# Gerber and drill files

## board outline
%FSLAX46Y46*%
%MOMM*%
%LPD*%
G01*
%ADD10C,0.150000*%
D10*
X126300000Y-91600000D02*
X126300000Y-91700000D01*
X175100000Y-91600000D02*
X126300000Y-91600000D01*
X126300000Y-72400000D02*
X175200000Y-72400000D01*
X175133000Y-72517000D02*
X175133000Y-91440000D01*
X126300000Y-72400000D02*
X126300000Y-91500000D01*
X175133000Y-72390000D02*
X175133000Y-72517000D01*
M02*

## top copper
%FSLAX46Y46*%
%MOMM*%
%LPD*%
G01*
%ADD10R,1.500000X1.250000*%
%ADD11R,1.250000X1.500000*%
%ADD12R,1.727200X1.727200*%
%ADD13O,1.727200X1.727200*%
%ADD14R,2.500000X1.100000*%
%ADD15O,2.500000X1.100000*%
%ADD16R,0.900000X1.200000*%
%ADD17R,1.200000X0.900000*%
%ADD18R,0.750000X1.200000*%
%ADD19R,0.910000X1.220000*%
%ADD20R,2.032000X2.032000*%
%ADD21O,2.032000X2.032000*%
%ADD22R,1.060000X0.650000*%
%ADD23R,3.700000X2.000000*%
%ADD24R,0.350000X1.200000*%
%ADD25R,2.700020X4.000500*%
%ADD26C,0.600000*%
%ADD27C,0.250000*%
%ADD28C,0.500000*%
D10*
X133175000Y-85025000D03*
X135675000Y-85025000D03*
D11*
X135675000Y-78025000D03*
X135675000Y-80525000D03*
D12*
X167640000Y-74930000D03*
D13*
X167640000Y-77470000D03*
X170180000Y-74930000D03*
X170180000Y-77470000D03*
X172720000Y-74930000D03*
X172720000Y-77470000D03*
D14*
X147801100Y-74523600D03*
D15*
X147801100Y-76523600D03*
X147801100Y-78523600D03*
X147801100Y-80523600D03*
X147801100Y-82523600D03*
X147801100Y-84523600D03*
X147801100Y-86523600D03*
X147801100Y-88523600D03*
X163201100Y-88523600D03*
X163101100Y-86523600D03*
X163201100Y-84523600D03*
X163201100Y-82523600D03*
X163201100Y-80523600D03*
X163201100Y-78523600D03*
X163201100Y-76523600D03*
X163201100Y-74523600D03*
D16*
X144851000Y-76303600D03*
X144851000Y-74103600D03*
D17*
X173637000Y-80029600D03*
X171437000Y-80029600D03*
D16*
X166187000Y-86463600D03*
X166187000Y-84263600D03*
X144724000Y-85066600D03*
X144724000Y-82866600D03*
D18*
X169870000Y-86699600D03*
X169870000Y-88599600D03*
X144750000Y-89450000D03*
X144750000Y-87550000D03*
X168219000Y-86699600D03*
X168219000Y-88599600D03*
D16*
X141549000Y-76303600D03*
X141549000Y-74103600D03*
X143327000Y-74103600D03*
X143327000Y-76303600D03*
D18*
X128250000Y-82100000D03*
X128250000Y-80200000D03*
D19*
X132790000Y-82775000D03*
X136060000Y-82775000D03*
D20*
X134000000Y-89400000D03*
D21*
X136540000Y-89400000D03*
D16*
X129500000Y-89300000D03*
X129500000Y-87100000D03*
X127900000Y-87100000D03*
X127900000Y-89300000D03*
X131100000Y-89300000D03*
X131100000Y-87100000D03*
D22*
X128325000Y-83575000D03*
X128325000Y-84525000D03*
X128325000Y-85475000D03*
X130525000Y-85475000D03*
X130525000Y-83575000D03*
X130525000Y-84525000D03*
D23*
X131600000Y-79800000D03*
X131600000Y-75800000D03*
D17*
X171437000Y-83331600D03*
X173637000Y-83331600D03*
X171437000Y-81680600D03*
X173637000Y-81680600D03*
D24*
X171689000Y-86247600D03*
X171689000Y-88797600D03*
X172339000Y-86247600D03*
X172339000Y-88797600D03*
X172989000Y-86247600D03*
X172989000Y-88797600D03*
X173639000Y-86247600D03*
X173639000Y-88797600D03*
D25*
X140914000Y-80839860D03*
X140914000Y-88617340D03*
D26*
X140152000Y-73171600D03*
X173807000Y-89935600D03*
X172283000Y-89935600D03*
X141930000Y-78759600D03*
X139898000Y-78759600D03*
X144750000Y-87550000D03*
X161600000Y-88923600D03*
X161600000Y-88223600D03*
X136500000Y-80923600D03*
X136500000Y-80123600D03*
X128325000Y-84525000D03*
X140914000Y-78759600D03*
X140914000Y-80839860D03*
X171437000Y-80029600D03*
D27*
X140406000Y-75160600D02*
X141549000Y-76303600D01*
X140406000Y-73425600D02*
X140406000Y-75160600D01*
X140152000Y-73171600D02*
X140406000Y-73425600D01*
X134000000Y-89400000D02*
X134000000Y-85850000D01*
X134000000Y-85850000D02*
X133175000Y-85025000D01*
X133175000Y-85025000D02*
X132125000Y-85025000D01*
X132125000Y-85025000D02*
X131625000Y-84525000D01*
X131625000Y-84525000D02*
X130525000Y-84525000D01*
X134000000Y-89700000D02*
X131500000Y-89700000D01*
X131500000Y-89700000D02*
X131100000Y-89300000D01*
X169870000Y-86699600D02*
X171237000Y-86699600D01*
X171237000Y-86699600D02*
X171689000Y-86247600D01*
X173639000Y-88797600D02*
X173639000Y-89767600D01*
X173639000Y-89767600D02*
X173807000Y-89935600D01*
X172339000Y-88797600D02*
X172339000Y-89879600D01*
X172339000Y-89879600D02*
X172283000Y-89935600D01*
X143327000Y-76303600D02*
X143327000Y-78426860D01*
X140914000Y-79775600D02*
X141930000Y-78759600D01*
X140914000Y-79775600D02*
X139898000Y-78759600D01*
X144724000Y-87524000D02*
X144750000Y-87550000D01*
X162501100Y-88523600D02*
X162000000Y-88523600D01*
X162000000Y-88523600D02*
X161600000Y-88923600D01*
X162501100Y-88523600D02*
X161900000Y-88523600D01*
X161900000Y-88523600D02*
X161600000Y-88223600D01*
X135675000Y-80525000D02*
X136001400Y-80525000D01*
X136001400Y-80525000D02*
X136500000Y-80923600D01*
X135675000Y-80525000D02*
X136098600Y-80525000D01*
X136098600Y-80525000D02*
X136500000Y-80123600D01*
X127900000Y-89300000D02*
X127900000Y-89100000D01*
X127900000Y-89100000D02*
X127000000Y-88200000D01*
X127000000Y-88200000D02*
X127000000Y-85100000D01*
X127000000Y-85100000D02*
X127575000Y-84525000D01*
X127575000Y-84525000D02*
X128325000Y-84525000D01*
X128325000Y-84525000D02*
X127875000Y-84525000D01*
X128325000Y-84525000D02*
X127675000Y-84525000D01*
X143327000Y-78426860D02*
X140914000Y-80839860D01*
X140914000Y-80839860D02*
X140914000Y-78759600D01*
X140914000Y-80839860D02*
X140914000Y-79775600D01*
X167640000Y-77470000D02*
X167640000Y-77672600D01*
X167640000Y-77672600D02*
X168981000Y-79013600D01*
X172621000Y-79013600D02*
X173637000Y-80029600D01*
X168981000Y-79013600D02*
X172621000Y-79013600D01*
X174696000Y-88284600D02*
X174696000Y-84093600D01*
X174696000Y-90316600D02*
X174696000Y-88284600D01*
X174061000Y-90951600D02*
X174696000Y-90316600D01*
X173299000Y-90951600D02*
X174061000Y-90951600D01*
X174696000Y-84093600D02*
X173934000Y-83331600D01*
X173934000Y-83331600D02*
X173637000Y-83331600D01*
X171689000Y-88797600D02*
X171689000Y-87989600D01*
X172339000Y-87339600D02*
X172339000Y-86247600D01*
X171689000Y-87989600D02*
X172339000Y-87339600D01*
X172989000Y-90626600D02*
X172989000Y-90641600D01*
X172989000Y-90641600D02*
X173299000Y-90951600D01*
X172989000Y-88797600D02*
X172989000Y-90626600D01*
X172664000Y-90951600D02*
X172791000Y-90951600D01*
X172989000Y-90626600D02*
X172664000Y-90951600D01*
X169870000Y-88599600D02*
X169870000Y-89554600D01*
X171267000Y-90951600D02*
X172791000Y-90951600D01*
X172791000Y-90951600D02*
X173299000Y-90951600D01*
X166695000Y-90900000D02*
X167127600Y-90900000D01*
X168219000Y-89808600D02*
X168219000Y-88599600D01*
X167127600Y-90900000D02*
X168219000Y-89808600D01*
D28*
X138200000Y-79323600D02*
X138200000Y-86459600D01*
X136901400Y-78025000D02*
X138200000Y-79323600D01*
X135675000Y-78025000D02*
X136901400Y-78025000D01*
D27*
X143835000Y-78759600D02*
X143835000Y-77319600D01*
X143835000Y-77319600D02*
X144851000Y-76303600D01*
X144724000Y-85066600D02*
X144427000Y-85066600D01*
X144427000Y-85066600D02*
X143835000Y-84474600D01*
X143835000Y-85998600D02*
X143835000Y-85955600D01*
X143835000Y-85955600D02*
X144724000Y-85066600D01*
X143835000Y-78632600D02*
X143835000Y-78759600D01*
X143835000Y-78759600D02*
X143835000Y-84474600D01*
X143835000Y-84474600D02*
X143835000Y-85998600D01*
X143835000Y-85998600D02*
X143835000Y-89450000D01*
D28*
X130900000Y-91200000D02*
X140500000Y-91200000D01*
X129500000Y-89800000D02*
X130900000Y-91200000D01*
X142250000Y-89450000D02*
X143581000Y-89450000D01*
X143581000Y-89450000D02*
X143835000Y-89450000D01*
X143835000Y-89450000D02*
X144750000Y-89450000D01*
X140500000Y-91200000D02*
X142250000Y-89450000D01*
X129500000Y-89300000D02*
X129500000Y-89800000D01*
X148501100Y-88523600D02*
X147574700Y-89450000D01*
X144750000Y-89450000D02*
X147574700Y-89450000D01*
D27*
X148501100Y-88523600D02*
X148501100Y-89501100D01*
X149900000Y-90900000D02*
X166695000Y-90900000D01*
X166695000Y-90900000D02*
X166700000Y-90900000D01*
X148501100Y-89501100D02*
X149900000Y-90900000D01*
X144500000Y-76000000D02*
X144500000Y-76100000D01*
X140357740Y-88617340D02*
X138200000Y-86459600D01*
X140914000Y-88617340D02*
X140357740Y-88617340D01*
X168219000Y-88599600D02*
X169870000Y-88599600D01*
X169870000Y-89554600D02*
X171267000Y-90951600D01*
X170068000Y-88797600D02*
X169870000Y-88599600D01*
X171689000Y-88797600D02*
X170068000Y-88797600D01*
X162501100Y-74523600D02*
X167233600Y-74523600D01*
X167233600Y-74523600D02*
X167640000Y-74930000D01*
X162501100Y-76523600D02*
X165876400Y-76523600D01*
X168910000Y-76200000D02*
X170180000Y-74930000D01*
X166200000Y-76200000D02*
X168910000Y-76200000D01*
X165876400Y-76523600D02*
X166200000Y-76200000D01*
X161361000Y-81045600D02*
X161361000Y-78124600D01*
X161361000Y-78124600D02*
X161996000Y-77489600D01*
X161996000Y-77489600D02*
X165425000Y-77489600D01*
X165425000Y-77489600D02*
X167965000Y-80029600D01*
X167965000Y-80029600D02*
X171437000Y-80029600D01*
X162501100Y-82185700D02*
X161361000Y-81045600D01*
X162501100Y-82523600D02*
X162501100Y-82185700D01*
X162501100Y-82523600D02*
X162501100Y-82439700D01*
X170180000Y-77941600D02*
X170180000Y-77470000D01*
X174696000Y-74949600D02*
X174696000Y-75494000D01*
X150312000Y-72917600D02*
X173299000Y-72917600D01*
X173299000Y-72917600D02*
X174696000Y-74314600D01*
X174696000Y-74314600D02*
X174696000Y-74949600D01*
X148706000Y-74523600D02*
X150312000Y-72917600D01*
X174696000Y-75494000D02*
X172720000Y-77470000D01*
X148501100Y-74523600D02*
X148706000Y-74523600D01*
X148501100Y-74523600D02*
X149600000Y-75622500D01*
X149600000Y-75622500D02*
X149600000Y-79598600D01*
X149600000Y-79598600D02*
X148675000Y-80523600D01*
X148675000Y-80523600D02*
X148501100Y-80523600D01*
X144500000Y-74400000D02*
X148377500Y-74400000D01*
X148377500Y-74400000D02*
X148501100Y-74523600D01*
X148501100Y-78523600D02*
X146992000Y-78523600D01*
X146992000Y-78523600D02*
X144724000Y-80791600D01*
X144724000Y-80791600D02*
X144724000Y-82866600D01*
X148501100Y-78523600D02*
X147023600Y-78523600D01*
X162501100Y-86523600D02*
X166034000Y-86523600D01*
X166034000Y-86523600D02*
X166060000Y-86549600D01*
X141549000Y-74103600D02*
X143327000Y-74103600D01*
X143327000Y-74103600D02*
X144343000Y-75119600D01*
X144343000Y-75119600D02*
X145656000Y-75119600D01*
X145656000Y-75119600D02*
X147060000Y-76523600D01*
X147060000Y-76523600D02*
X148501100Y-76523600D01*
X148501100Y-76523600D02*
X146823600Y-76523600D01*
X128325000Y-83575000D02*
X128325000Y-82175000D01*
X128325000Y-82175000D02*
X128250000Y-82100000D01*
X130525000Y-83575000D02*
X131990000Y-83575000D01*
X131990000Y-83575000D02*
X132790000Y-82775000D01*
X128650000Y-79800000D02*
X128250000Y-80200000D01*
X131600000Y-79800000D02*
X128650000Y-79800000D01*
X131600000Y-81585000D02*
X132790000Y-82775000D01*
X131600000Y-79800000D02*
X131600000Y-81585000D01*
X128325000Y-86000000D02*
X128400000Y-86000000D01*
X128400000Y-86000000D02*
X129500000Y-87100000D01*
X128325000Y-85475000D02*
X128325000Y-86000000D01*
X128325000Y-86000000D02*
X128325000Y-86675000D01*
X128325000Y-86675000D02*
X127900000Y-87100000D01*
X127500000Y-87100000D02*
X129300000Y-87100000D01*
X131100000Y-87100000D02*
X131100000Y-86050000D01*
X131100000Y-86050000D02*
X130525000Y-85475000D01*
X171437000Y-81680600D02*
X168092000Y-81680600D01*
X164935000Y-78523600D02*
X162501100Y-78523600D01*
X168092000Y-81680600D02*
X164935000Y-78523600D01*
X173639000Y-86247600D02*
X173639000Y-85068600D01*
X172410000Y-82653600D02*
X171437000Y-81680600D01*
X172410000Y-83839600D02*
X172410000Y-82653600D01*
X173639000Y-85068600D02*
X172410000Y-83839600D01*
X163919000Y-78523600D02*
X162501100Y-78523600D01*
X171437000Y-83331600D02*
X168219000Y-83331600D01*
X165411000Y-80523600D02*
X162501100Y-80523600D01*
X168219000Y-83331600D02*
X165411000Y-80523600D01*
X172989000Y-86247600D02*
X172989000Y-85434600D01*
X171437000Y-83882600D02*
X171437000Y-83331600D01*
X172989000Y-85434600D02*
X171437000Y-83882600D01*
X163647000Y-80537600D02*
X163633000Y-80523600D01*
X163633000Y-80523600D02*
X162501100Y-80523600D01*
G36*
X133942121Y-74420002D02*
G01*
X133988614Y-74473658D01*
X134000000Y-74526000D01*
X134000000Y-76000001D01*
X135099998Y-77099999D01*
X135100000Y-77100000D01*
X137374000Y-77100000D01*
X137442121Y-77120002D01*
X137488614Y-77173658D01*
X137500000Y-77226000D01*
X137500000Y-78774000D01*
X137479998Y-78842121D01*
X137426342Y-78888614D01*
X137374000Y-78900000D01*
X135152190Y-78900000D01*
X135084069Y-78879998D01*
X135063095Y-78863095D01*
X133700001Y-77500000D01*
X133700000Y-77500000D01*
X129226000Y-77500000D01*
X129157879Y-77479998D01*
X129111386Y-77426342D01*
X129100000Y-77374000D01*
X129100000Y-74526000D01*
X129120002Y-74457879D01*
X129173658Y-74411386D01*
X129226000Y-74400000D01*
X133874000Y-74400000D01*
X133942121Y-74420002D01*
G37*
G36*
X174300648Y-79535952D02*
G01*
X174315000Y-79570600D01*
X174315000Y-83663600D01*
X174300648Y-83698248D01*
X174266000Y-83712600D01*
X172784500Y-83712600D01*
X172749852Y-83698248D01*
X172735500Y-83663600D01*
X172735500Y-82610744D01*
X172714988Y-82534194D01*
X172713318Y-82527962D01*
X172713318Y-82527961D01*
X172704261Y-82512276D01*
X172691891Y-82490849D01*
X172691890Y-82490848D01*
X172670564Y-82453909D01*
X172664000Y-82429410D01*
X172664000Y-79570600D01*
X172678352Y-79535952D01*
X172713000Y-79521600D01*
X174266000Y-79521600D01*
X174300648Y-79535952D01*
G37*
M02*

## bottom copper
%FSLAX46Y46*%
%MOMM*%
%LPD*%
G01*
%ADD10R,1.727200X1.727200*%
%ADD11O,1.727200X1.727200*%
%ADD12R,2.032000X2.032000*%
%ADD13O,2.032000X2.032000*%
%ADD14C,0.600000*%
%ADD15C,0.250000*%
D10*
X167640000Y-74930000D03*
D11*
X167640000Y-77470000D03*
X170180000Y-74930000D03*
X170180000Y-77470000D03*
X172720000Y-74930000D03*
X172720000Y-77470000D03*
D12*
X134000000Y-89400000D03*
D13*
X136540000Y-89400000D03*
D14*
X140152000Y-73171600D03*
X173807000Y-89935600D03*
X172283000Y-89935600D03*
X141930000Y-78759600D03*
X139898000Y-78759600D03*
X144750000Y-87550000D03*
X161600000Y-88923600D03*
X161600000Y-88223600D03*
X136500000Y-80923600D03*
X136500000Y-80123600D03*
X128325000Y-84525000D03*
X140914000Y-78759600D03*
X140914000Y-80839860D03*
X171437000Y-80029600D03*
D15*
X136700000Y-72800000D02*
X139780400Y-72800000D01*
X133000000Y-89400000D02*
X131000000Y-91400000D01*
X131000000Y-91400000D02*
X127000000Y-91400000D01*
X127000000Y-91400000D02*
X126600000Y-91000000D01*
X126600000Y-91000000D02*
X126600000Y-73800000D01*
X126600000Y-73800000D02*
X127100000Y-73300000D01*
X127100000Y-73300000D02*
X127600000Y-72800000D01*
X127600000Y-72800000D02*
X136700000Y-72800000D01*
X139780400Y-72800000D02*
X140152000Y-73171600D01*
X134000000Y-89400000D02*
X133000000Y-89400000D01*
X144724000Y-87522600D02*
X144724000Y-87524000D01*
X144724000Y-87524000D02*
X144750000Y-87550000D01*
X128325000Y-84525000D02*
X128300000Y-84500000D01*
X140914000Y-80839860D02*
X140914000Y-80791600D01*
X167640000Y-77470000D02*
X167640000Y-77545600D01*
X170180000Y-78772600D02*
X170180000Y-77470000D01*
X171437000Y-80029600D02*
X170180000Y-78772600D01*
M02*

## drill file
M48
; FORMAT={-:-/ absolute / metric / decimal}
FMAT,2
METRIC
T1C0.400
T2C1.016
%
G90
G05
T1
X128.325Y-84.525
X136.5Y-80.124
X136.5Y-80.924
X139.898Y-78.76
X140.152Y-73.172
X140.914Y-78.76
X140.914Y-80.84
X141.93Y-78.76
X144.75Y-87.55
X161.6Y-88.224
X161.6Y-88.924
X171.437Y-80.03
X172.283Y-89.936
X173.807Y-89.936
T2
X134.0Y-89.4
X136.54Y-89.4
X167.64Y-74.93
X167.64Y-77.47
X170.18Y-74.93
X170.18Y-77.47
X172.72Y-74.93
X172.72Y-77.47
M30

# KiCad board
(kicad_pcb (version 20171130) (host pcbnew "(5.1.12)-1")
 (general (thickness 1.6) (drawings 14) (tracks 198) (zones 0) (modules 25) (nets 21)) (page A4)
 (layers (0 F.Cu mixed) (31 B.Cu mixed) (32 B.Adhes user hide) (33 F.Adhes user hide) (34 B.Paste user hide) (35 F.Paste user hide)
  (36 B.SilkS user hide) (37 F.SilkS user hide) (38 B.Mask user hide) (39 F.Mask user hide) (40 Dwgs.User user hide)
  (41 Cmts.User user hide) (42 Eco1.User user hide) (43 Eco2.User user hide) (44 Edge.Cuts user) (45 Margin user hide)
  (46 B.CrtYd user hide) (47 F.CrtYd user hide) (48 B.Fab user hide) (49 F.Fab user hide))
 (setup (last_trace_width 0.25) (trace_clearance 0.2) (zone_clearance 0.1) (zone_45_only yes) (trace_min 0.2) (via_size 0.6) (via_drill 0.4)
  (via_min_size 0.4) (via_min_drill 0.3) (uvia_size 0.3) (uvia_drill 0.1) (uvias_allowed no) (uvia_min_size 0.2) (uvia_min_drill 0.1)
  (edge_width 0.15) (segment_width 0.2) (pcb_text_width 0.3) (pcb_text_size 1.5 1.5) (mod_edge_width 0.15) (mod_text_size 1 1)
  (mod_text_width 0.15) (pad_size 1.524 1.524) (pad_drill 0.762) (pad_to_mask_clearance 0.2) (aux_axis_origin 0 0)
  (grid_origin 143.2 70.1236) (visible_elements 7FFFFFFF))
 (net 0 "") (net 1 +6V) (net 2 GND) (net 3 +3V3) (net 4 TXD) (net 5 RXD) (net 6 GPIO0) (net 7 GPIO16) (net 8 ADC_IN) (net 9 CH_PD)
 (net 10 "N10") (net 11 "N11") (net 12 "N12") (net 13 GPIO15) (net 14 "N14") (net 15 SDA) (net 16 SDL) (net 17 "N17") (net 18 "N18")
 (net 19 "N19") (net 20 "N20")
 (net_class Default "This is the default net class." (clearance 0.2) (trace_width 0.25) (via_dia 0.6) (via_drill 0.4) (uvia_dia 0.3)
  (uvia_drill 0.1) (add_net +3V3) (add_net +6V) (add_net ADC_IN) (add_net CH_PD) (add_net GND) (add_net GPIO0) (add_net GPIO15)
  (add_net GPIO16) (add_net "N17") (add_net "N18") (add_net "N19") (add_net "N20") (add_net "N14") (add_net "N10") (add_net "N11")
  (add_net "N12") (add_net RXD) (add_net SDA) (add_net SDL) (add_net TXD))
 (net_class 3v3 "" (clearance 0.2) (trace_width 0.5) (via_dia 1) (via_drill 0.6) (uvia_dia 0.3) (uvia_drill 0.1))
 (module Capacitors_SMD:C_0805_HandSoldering (layer F.Cu) (at 134.425 85.025)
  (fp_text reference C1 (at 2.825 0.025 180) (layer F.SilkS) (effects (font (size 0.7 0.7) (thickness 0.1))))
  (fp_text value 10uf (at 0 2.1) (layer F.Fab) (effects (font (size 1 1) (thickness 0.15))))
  (pad 1 smd rect (at -1.25 0) (size 1.5 1.25) (layers F.Cu F.Paste F.Mask) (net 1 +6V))
  (pad 2 smd rect (at 1.25 0) (size 1.5 1.25) (layers F.Cu F.Paste F.Mask) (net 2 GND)))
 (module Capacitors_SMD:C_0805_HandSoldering (layer F.Cu) (at 135.675 79.275 270)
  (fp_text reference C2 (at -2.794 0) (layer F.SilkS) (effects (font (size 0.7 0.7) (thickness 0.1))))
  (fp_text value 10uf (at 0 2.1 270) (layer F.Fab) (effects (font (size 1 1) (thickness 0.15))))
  (pad 1 smd rect (at -1.25 0 270) (size 1.5 1.25) (layers F.Cu F.Paste F.Mask) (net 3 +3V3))
  (pad 2 smd rect (at 1.25 0 270) (size 1.5 1.25) (layers F.Cu F.Paste F.Mask) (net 2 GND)))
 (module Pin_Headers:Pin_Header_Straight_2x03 (layer B.Cu) (at 167.64 74.93 270)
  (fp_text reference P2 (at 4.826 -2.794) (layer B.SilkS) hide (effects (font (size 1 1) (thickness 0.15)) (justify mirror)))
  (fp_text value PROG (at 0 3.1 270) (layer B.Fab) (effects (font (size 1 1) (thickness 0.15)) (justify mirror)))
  (pad 1 thru_hole rect (at 0 0 270) (size 1.7272 1.7272) (drill 1.016) (layers *.Cu *.Mask B.SilkS) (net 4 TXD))
  (pad 2 thru_hole oval (at 2.54 0 270) (size 1.7272 1.7272) (drill 1.016) (layers *.Cu *.Mask B.SilkS) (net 3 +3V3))
  (pad 3 thru_hole oval (at 0 -2.54 270) (size 1.7272 1.7272) (drill 1.016) (layers *.Cu *.Mask B.SilkS) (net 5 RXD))
  (pad 4 thru_hole oval (at 2.54 -2.54 270) (size 1.7272 1.7272) (drill 1.016) (layers *.Cu *.Mask B.SilkS) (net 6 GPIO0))
  (pad 5 thru_hole oval (at 0 -5.08 270) (size 1.7272 1.7272) (drill 1.016) (layers *.Cu *.Mask B.SilkS) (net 2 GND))
  (pad 6 thru_hole oval (at 2.54 -5.08 270) (size 1.7272 1.7272) (drill 1.016) (layers *.Cu *.Mask B.SilkS) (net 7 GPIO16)))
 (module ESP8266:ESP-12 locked (layer F.Cu) (at 148.5011 74.5236)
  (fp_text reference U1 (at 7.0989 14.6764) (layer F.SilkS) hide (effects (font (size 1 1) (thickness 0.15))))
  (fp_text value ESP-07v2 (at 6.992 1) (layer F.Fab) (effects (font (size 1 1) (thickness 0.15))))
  (pad 1 smd rect (at 0 0) (size 2.5 1.1) (drill (offset -0.7 0)) (layers F.Cu F.Paste F.Mask) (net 7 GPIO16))
  (pad 2 smd oval (at 0 2) (size 2.5 1.1) (drill (offset -0.7 0)) (layers F.Cu F.Paste F.Mask) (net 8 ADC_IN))
  (pad 3 smd oval (at 0 4) (size 2.5 1.1) (drill (offset -0.7 0)) (layers F.Cu F.Paste F.Mask) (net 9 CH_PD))
  (pad 4 smd oval (at 0 6) (size 2.5 1.1) (drill (offset -0.7 0)) (layers F.Cu F.Paste F.Mask) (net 7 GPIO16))
  (pad 5 smd oval (at 0 8) (size 2.5 1.1) (drill (offset -0.7 0)) (layers F.Cu F.Paste F.Mask) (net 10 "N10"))
  (pad 6 smd oval (at 0 10) (size 2.5 1.1) (drill (offset -0.7 0)) (layers F.Cu F.Paste F.Mask) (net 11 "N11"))
  (pad 7 smd oval (at 0 12) (size 2.5 1.1) (drill (offset -0.7 0)) (layers F.Cu F.Paste F.Mask) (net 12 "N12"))
  (pad 8 smd oval (at 0 14) (size 2.5 1.1) (drill (offset -0.7 0)) (layers F.Cu F.Paste F.Mask) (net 3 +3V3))
  (pad 9 smd oval (at 14 14) (size 2.5 1.1) (drill (offset 0.7 0)) (layers F.Cu F.Paste F.Mask) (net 2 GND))
  (pad 10 smd oval (at 14 12) (size 2.5 1.1) (drill (offset 0.6 0)) (layers F.Cu F.Paste F.Mask) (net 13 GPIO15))
  (pad 11 smd oval (at 14 10) (size 2.5 1.1) (drill (offset 0.7 0)) (layers F.Cu F.Paste F.Mask) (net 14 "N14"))
  (pad 12 smd oval (at 14 8) (size 2.5 1.1) (drill (offset 0.7 0)) (layers F.Cu F.Paste F.Mask) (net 6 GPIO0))
  (pad 13 smd oval (at 14 6) (size 2.5 1.1) (drill (offset 0.7 0)) (layers F.Cu F.Paste F.Mask) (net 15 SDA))
  (pad 14 smd oval (at 14 4) (size 2.5 1.1) (drill (offset 0.7 0)) (layers F.Cu F.Paste F.Mask) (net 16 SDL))
  (pad 15 smd oval (at 14 2) (size 2.5 1.1) (drill (offset 0.7 0)) (layers F.Cu F.Paste F.Mask) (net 5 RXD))
  (pad 16 smd oval (at 14 0) (size 2.5 1.1) (drill (offset 0.7 0)) (layers F.Cu F.Paste F.Mask) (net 4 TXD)))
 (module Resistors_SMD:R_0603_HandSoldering (layer F.Cu) (at 144.851 75.2036 90)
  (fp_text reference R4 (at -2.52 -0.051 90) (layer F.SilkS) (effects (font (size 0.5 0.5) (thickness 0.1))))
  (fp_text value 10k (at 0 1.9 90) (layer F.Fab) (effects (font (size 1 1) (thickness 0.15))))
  (pad 1 smd rect (at -1.1 0 90) (size 1.2 0.9) (layers F.Cu F.Paste F.Mask) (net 3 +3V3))
  (pad 2 smd rect (at 1.1 0 90) (size 1.2 0.9) (layers F.Cu F.Paste F.Mask) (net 7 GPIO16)))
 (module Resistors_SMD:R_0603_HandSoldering (layer F.Cu) (at 172.537 80.0296 180)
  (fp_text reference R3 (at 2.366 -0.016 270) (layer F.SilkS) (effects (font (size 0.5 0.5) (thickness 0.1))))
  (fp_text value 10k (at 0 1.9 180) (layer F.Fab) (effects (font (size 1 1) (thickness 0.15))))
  (pad 1 smd rect (at -1.1 0 180) (size 1.2 0.9) (layers F.Cu F.Paste F.Mask) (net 3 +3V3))
  (pad 2 smd rect (at 1.1 0 180) (size 1.2 0.9) (layers F.Cu F.Paste F.Mask) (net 6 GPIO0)))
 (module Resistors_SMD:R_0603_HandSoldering (layer F.Cu) (at 166.187 85.3636 90)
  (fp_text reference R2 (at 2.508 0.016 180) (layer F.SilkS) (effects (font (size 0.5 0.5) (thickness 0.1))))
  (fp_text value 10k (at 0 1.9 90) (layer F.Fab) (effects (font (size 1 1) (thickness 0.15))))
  (pad 1 smd rect (at -1.1 0 90) (size 1.2 0.9) (layers F.Cu F.Paste F.Mask) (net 13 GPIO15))
  (pad 2 smd rect (at 1.1 0 90) (size 1.2 0.9) (layers F.Cu F.Paste F.Mask) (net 2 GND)))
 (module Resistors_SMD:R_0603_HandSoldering (layer F.Cu) (at 144.724 83.9666 90)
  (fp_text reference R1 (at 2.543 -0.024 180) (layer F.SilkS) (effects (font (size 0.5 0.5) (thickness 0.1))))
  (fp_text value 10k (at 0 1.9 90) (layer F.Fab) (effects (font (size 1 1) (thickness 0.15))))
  (pad 1 smd rect (at -1.1 0 90) (size 1.2 0.9) (layers F.Cu F.Paste F.Mask) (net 3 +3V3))
  (pad 2 smd rect (at 1.1 0 90) (size 1.2 0.9) (layers F.Cu F.Paste F.Mask) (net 9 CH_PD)))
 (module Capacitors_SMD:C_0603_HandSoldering (layer F.Cu) (at 169.87 87.6496 270)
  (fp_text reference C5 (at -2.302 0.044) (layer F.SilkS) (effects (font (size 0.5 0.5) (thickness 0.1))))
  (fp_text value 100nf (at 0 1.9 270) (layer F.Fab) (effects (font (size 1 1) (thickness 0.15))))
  (pad 1 smd rect (at -0.95 0 270) (size 1.2 0.75) (layers F.Cu F.Paste F.Mask) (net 2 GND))
  (pad 2 smd rect (at 0.95 0 270) (size 1.2 0.75) (layers F.Cu F.Paste F.Mask) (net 3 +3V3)))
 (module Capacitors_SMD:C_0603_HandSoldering (layer F.Cu) (at 144.75 88.5 90)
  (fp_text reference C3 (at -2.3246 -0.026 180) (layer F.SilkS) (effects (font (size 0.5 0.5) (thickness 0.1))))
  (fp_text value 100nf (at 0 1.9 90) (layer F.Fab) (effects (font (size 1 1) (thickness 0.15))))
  (pad 1 smd rect (at -0.95 0 90) (size 1.2 0.75) (layers F.Cu F.Paste F.Mask) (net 3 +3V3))
  (pad 2 smd rect (at 0.95 0 90) (size 1.2 0.75) (layers F.Cu F.Paste F.Mask) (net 2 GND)))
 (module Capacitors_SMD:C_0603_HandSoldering (layer F.Cu) (at 168.219 87.6496 270)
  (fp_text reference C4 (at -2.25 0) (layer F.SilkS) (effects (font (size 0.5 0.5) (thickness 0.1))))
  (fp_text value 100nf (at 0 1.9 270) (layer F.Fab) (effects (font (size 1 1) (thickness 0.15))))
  (pad 1 smd rect (at -0.95 0 270) (size 1.2 0.75) (layers F.Cu F.Paste F.Mask) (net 2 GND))
  (pad 2 smd rect (at 0.95 0 270) (size 1.2 0.75) (layers F.Cu F.Paste F.Mask) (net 3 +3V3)))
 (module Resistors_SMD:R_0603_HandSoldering (layer F.Cu) (at 141.549 75.2036 90)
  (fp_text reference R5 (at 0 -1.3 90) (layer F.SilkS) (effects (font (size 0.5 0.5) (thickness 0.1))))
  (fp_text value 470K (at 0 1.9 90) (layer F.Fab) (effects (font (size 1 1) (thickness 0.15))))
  (pad 1 smd rect (at -1.1 0 90) (size 1.2 0.9) (layers F.Cu F.Paste F.Mask) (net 1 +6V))
  (pad 2 smd rect (at 1.1 0 90) (size 1.2 0.9) (layers F.Cu F.Paste F.Mask) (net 8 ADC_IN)))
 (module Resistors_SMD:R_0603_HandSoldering (layer F.Cu) (at 143.327 75.2036 270)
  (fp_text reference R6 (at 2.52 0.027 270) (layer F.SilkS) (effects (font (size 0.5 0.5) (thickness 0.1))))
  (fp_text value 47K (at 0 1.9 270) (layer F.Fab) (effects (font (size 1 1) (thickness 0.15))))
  (pad 1 smd rect (at -1.1 0 270) (size 1.2 0.9) (layers F.Cu F.Paste F.Mask) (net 8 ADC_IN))
  (pad 2 smd rect (at 1.1 0 270) (size 1.2 0.9) (layers F.Cu F.Paste F.Mask) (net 2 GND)))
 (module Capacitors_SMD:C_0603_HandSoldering (layer F.Cu) (at 128.25 81.15 90)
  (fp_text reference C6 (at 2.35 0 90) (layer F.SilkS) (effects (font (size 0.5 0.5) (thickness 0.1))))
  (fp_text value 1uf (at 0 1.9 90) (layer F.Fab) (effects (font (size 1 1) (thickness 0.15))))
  (pad 1 smd rect (at -0.95 0 90) (size 1.2 0.75) (layers F.Cu F.Paste F.Mask) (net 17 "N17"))
  (pad 2 smd rect (at 0.95 0 90) (size 1.2 0.75) (layers F.Cu F.Paste F.Mask) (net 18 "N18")))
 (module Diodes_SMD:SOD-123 (layer F.Cu) (at 134.425 82.775)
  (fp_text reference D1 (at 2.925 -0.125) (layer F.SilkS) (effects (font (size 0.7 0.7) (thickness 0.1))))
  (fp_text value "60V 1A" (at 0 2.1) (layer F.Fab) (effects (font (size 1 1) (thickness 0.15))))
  (pad 1 smd rect (at -1.635 0) (size 0.91 1.22) (layers F.Cu F.Paste F.Mask) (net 18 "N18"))
  (pad 2 smd rect (at 1.635 0) (size 0.91 1.22) (layers F.Cu F.Paste F.Mask) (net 2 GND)))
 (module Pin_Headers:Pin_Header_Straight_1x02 (layer F.Cu) (at 134 89.4 90)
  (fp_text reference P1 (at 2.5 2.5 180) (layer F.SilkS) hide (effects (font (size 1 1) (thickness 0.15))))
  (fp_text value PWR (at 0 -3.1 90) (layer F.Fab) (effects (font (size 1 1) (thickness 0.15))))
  (pad 1 thru_hole rect (at 0 0 90) (size 2.032 2.032) (drill 1.016) (layers *.Cu *.Mask F.SilkS) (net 1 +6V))
  (pad 2 thru_hole oval (at 0 2.54 90) (size 2.032 2.032) (drill 1.016) (layers *.Cu *.Mask F.SilkS) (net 2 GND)))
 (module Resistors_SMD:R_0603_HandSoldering (layer F.Cu) (at 129.5 88.2 90)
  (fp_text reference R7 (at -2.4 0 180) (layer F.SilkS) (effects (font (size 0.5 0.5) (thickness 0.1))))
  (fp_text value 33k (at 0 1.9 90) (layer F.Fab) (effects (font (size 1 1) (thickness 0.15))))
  (pad 1 smd rect (at -1.1 0 90) (size 1.2 0.9) (layers F.Cu F.Paste F.Mask) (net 3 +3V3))
  (pad 2 smd rect (at 1.1 0 90) (size 1.2 0.9) (layers F.Cu F.Paste F.Mask) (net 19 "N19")))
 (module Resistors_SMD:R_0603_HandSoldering (layer F.Cu) (at 127.9 88.2 270)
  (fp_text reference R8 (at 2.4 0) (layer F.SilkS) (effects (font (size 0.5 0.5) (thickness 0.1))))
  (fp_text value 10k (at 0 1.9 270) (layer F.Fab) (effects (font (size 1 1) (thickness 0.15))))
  (pad 1 smd rect (at -1.1 0 270) (size 1.2 0.9) (layers F.Cu F.Paste F.Mask) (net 19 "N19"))
  (pad 2 smd rect (at 1.1 0 270) (size 1.2 0.9) (layers F.Cu F.Paste F.Mask) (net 2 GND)))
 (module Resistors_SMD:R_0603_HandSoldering (layer F.Cu) (at 131.1 88.2 90)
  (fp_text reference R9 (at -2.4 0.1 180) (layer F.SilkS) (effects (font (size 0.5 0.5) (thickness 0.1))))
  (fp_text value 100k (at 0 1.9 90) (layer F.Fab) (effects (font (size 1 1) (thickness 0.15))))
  (pad 1 smd rect (at -1.1 0 90) (size 1.2 0.9) (layers F.Cu F.Paste F.Mask) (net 1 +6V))
  (pad 2 smd rect (at 1.1 0 90) (size 1.2 0.9) (layers F.Cu F.Paste F.Mask) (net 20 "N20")))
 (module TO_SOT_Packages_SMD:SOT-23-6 (layer F.Cu) (at 129.425 84.525) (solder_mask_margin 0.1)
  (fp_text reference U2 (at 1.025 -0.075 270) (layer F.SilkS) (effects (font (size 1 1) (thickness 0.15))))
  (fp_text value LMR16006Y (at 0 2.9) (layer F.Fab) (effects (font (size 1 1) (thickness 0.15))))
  (pad 1 smd rect (at -1.1 -0.95) (size 1.06 0.65) (layers F.Cu F.Paste F.Mask) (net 17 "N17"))
  (pad 2 smd rect (at -1.1 0) (size 1.06 0.65) (layers F.Cu F.Paste F.Mask) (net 2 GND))
  (pad 3 smd rect (at -1.1 0.95) (size 1.06 0.65) (layers F.Cu F.Paste F.Mask) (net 19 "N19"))
  (pad 4 smd rect (at 1.1 0.95) (size 1.06 0.65) (layers F.Cu F.Paste F.Mask) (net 20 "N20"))
  (pad 6 smd rect (at 1.1 -0.95) (size 1.06 0.65) (layers F.Cu F.Paste F.Mask) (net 18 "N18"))
  (pad 5 smd rect (at 1.1 0) (size 1.06 0.65) (layers F.Cu F.Paste F.Mask) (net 1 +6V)))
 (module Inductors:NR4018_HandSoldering (layer F.Cu) (at 131.6 77.8 90)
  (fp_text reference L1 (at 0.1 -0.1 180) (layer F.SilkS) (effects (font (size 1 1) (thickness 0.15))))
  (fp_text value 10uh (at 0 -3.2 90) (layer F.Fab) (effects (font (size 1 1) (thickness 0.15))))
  (pad 1 smd rect (at -2 0 90) (size 2 3.7) (layers F.Cu F.Paste F.Mask) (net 18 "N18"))
  (pad 2 smd rect (at 2 0 90) (size 2 3.7) (layers F.Cu F.Paste F.Mask) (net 3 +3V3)))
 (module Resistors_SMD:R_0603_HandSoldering (layer F.Cu) (at 172.537 83.3316)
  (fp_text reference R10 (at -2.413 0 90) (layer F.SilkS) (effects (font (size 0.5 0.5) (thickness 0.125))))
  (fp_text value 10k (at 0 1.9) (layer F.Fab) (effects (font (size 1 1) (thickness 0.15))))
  (pad 1 smd rect (at -1.1 0) (size 1.2 0.9) (layers F.Cu F.Paste F.Mask) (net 15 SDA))
  (pad 2 smd rect (at 1.1 0) (size 1.2 0.9) (layers F.Cu F.Paste F.Mask) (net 3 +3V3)))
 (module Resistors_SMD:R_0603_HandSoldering (layer F.Cu) (at 172.537 81.6806)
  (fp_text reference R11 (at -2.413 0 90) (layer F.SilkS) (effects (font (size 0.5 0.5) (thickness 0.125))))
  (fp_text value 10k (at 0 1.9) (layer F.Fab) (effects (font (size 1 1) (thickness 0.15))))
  (pad 1 smd rect (at -1.1 0) (size 1.2 0.9) (layers F.Cu F.Paste F.Mask) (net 16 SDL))
  (pad 2 smd rect (at 1.1 0) (size 1.2 0.9) (layers F.Cu F.Paste F.Mask) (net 3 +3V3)))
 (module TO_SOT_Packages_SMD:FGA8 (layer F.Cu) (at 172.664 87.5226)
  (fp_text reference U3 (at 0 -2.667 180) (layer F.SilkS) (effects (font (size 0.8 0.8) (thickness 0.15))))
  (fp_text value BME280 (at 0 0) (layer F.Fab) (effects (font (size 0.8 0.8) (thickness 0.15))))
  (pad 1 smd rect (at -0.975 -1.275) (size 0.35 1.2) (layers F.Cu F.Paste F.Mask) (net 2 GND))
  (pad 8 smd rect (at -0.975 1.275) (size 0.35 1.2) (layers F.Cu F.Paste F.Mask) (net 3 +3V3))
  (pad 2 smd rect (at -0.325 -1.275) (size 0.35 1.2) (layers F.Cu F.Paste F.Mask) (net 3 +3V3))
  (pad 7 smd rect (at -0.325 1.275) (size 0.35 1.2) (layers F.Cu F.Paste F.Mask) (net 2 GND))
  (pad 3 smd rect (at 0.325 -1.275) (size 0.35 1.2) (layers F.Cu F.Paste F.Mask) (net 15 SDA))
  (pad 6 smd rect (at 0.325 1.275) (size 0.35 1.2) (layers F.Cu F.Paste F.Mask) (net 3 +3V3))
  (pad 4 smd rect (at 0.975 -1.275) (size 0.35 1.2) (layers F.Cu F.Paste F.Mask) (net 16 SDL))
  (pad 5 smd rect (at 0.975 1.275) (size 0.35 1.2) (layers F.Cu F.Paste F.Mask) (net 2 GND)))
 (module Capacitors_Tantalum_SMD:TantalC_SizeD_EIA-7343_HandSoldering (layer F.Cu) (at 140.914 84.7286 90)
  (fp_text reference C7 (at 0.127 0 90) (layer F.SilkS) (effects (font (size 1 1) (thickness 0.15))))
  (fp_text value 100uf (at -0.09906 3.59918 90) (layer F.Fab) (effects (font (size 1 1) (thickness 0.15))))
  (pad 2 smd rect (at 3.88874 0 90) (size 4.0005 2.70002) (layers F.Cu F.Paste F.Mask) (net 2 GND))
  (pad 1 smd rect (at -3.88874 0 90) (size 4.0005 2.70002) (layers F.Cu F.Paste F.Mask) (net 3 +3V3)))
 (gr_line (start 126.3 91.6) (end 126.3 91.7) (angle 90) (layer Edge.Cuts) (width 0.15))
 (gr_line (start 175.1 91.6) (end 126.3 91.6) (angle 90) (layer Edge.Cuts) (width 0.15))
 (gr_line (start 126.3 72.4) (end 175.2 72.4) (angle 90) (layer Edge.Cuts) (width 0.15))
 (gr_line (start 175.133 72.517) (end 175.133 91.44) (angle 90) (layer Edge.Cuts) (width 0.15))
 (gr_line (start 126.3 72.4) (end 126.3 91.5) (angle 90) (layer Edge.Cuts) (width 0.15))
 (gr_line (start 175.133 72.39) (end 175.133 72.517) (angle 90) (layer Edge.Cuts) (width 0.15))
 (segment (start 136.7 72.8) (end 139.7804 72.8) (width 0.25) (layer B.Cu) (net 1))
 (segment (start 133 89.4) (end 131 91.4) (width 0.25) (layer B.Cu) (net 1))
 (segment (start 131 91.4) (end 127 91.4) (width 0.25) (layer B.Cu) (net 1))
 (segment (start 127 91.4) (end 126.6 91) (width 0.25) (layer B.Cu) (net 1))
 (segment (start 126.6 91) (end 126.6 73.8) (width 0.25) (layer B.Cu) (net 1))
 (segment (start 126.6 73.8) (end 127.1 73.3) (width 0.25) (layer B.Cu) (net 1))
 (segment (start 127.1 73.3) (end 127.6 72.8) (width 0.25) (layer B.Cu) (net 1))
 (segment (start 127.6 72.8) (end 136.7 72.8) (width 0.25) (layer B.Cu) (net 1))
 (segment (start 140.406 75.1606) (end 141.549 76.3036) (width 0.25) (layer F.Cu) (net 1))
 (segment (start 140.406 73.4256) (end 140.406 75.1606) (width 0.25) (layer F.Cu) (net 1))
 (segment (start 140.152 73.1716) (end 140.406 73.4256) (width 0.25) (layer F.Cu) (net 1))
 (via (at 140.152 73.1716) (size 0.6) (drill 0.4) (layers F.Cu B.Cu) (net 1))
 (segment (start 139.7804 72.8) (end 140.152 73.1716) (width 0.25) (layer B.Cu) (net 1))
 (segment (start 134 89.4) (end 134 85.85) (width 0.25) (layer F.Cu) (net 1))
 (segment (start 134 85.85) (end 133.175 85.025) (width 0.25) (layer F.Cu) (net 1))
 (segment (start 134 89.4) (end 133 89.4) (width 0.25) (layer B.Cu) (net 1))
 (segment (start 133.175 85.025) (end 132.125 85.025) (width 0.25) (layer F.Cu) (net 1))
 (segment (start 132.125 85.025) (end 131.625 84.525) (width 0.25) (layer F.Cu) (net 1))
 (segment (start 131.625 84.525) (end 130.525 84.525) (width 0.25) (layer F.Cu) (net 1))
 (segment (start 134 89.7) (end 131.5 89.7) (width 0.25) (layer F.Cu) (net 1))
 (segment (start 131.5 89.7) (end 131.1 89.3) (width 0.25) (layer F.Cu) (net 1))
 (segment (start 169.87 86.6996) (end 171.237 86.6996) (width 0.25) (layer F.Cu) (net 2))
 (segment (start 171.237 86.6996) (end 171.689 86.2476) (width 0.25) (layer F.Cu) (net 2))
 (segment (start 173.639 88.7976) (end 173.639 89.7676) (width 0.25) (layer F.Cu) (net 2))
 (via (at 173.807 89.9356) (size 0.6) (drill 0.4) (layers F.Cu B.Cu) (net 2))
 (segment (start 173.639 89.7676) (end 173.807 89.9356) (width 0.25) (layer F.Cu) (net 2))
 (segment (start 172.339 88.7976) (end 172.339 89.8796) (width 0.25) (layer F.Cu) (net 2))
 (via (at 172.283 89.9356) (size 0.6) (drill 0.4) (layers F.Cu B.Cu) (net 2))
 (segment (start 172.339 89.8796) (end 172.283 89.9356) (width 0.25) (layer F.Cu) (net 2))
 (segment (start 143.327 76.3036) (end 143.327 78.42686) (width 0.25) (layer F.Cu) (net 2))
 (segment (start 140.914 79.7756) (end 141.93 78.7596) (width 0.25) (layer F.Cu) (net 2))
 (via (at 141.93 78.7596) (size 0.6) (drill 0.4) (layers F.Cu B.Cu) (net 2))
 (segment (start 140.914 79.7756) (end 139.898 78.7596) (width 0.25) (layer F.Cu) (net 2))
 (via (at 139.898 78.7596) (size 0.6) (drill 0.4) (layers F.Cu B.Cu) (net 2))
 (segment (start 144.724 87.524) (end 144.75 87.55) (width 0.25) (layer F.Cu) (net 2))
 (via (at 144.75 87.55) (size 0.6) (drill 0.4) (layers F.Cu B.Cu) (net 2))
 (segment (start 144.724 87.5226) (end 144.724 87.524) (width 0.25) (layer B.Cu) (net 2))
 (segment (start 144.724 87.524) (end 144.75 87.55) (width 0.25) (layer B.Cu) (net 2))
 (segment (start 162.5011 88.5236) (end 162 88.5236) (width 0.25) (layer F.Cu) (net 2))
 (segment (start 162 88.5236) (end 161.6 88.9236) (width 0.25) (layer F.Cu) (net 2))
 (via (at 161.6 88.9236) (size 0.6) (drill 0.4) (layers F.Cu B.Cu) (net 2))
 (segment (start 162.5011 88.5236) (end 161.9 88.5236) (width 0.25) (layer F.Cu) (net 2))
 (via (at 161.6 88.2236) (size 0.6) (drill 0.4) (layers F.Cu B.Cu) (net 2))
 (segment (start 161.9 88.5236) (end 161.6 88.2236) (width 0.25) (layer F.Cu) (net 2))
 (segment (start 135.675 80.525) (end 136.0014 80.525) (width 0.25) (layer F.Cu) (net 2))
 (segment (start 136.0014 80.525) (end 136.5 80.9236) (width 0.25) (layer F.Cu) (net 2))
 (via (at 136.5 80.9236) (size 0.6) (drill 0.4) (layers F.Cu B.Cu) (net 2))
 (segment (start 135.675 80.525) (end 136.0986 80.525) (width 0.25) (layer F.Cu) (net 2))
 (segment (start 136.0986 80.525) (end 136.5 80.1236) (width 0.25) (layer F.Cu) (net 2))
 (via (at 136.5 80.1236) (size 0.6) (drill 0.4) (layers F.Cu B.Cu) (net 2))
 (via (at 128.325 84.525) (size 0.6) (drill 0.4) (layers F.Cu B.Cu) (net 2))
 (segment (start 128.325 84.525) (end 128.3 84.5) (width 0.25) (layer B.Cu) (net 2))
 (segment (start 127.9 89.3) (end 127.9 89.1) (width 0.25) (layer F.Cu) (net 2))
 (segment (start 127.9 89.1) (end 127 88.2) (width 0.25) (layer F.Cu) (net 2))
 (segment (start 127 88.2) (end 127 85.1) (width 0.25) (layer F.Cu) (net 2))
 (segment (start 127 85.1) (end 127.575 84.525) (width 0.25) (layer F.Cu) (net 2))
 (segment (start 127.575 84.525) (end 128.325 84.525) (width 0.25) (layer F.Cu) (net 2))
 (segment (start 128.325 84.525) (end 127.875 84.525) (width 0.25) (layer F.Cu) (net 2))
 (segment (start 128.325 84.525) (end 127.675 84.525) (width 0.25) (layer F.Cu) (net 2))
 (segment (start 143.327 78.42686) (end 140.914 80.83986) (width 0.25) (layer F.Cu) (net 2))
 (segment (start 140.914 80.83986) (end 140.914 78.7596) (width 0.25) (layer F.Cu) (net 2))
 (via (at 140.914 78.7596) (size 0.6) (drill 0.4) (layers F.Cu B.Cu) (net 2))
 (segment (start 140.914 80.83986) (end 140.914 79.7756) (width 0.25) (layer F.Cu) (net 2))
 (via (at 140.914 80.83986) (size 0.6) (drill 0.4) (layers F.Cu B.Cu) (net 2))
 (segment (start 140.914 80.83986) (end 140.914 80.7916) (width 0.25) (layer B.Cu) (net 2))
 (segment (start 167.64 77.47) (end 167.64 77.6726) (width 0.25) (layer F.Cu) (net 3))
 (segment (start 167.64 77.6726) (end 168.981 79.0136) (width 0.25) (layer F.Cu) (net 3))
 (segment (start 172.621 79.0136) (end 173.637 80.0296) (width 0.25) (layer F.Cu) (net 3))
 (segment (start 168.981 79.0136) (end 172.621 79.0136) (width 0.25) (layer F.Cu) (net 3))
 (segment (start 167.64 77.47) (end 167.64 77.5456) (width 0.25) (layer B.Cu) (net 3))
 (segment (start 174.696 88.2846) (end 174.696 84.0936) (width 0.25) (layer F.Cu) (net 3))
 (segment (start 174.696 90.3166) (end 174.696 88.2846) (width 0.25) (layer F.Cu) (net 3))
 (segment (start 174.061 90.9516) (end 174.696 90.3166) (width 0.25) (layer F.Cu) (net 3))
 (segment (start 173.299 90.9516) (end 174.061 90.9516) (width 0.25) (layer F.Cu) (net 3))
 (segment (start 174.696 84.0936) (end 173.934 83.3316) (width 0.25) (layer F.Cu) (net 3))
 (segment (start 173.934 83.3316) (end 173.637 83.3316) (width 0.25) (layer F.Cu) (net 3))
 (segment (start 171.689 88.7976) (end 171.689 87.9896) (width 0.25) (layer F.Cu) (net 3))
 (segment (start 172.339 87.3396) (end 172.339 86.2476) (width 0.25) (layer F.Cu) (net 3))
 (segment (start 171.689 87.9896) (end 172.339 87.3396) (width 0.25) (layer F.Cu) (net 3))
 (segment (start 172.989 90.6266) (end 172.989 90.6416) (width 0.25) (layer F.Cu) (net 3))
 (segment (start 172.989 90.6416) (end 173.299 90.9516) (width 0.25) (layer F.Cu) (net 3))
 (segment (start 172.989 88.7976) (end 172.989 90.6266) (width 0.25) (layer F.Cu) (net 3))
 (segment (start 172.664 90.9516) (end 172.791 90.9516) (width 0.25) (layer F.Cu) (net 3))
 (segment (start 172.989 90.6266) (end 172.664 90.9516) (width 0.25) (layer F.Cu) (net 3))
 (segment (start 169.87 88.5996) (end 169.87 89.5546) (width 0.25) (layer F.Cu) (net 3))
 (segment (start 171.267 90.9516) (end 172.791 90.9516) (width 0.25) (layer F.Cu) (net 3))
 (segment (start 172.791 90.9516) (end 173.299 90.9516) (width 0.25) (layer F.Cu) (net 3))
 (segment (start 166.695 90.9) (end 167.1276 90.9) (width 0.25) (layer F.Cu) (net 3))
 (segment (start 168.219 89.8086) (end 168.219 88.5996) (width 0.25) (layer F.Cu) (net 3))
 (segment (start 167.1276 90.9) (end 168.219 89.8086) (width 0.25) (layer F.Cu) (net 3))
 (segment (start 138.2 79.3236) (end 138.2 86.4596) (width 0.5) (layer F.Cu) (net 3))
 (segment (start 136.9014 78.025) (end 138.2 79.3236) (width 0.5) (layer F.Cu) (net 3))
 (segment (start 135.675 78.025) (end 136.9014 78.025) (width 0.5) (layer F.Cu) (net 3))
 (segment (start 143.835 78.7596) (end 143.835 77.3196) (width 0.25) (layer F.Cu) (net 3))
 (segment (start 143.835 77.3196) (end 144.851 76.3036) (width 0.25) (layer F.Cu) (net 3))
 (segment (start 144.724 85.0666) (end 144.427 85.0666) (width 0.25) (layer F.Cu) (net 3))
 (segment (start 144.427 85.0666) (end 143.835 84.4746) (width 0.25) (layer F.Cu) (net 3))
 (segment (start 143.835 85.9986) (end 143.835 85.9556) (width 0.25) (layer F.Cu) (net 3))
 (segment (start 143.835 85.9556) (end 144.724 85.0666) (width 0.25) (layer F.Cu) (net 3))
 (segment (start 143.835 78.6326) (end 143.835 78.7596) (width 0.25) (layer F.Cu) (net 3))
 (segment (start 143.835 78.7596) (end 143.835 84.4746) (width 0.25) (layer F.Cu) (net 3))
 (segment (start 143.835 84.4746) (end 143.835 85.9986) (width 0.25) (layer F.Cu) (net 3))
 (segment (start 143.835 85.9986) (end 143.835 89.45) (width 0.25) (layer F.Cu) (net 3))
 (segment (start 130.9 91.2) (end 140.5 91.2) (width 0.5) (layer F.Cu) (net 3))
 (segment (start 129.5 89.8) (end 130.9 91.2) (width 0.5) (layer F.Cu) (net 3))
 (segment (start 142.25 89.45) (end 143.581 89.45) (width 0.5) (layer F.Cu) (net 3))
 (segment (start 143.581 89.45) (end 143.835 89.45) (width 0.5) (layer F.Cu) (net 3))
 (segment (start 143.835 89.45) (end 144.75 89.45) (width 0.5) (layer F.Cu) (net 3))
 (segment (start 140.5 91.2) (end 142.25 89.45) (width 0.5) (layer F.Cu) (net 3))
 (segment (start 129.5 89.3) (end 129.5 89.8) (width 0.5) (layer F.Cu) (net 3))
 (segment (start 148.5011 88.5236) (end 147.5747 89.45) (width 0.5) (layer F.Cu) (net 3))
 (segment (start 144.75 89.45) (end 147.5747 89.45) (width 0.5) (layer F.Cu) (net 3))
 (segment (start 148.5011 88.5236) (end 148.5011 89.5011) (width 0.25) (layer F.Cu) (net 3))
 (segment (start 149.9 90.9) (end 166.695 90.9) (width 0.25) (layer F.Cu) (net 3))
 (segment (start 166.695 90.9) (end 166.7 90.9) (width 0.25) (layer F.Cu) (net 3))
 (segment (start 148.5011 89.5011) (end 149.9 90.9) (width 0.25) (layer F.Cu) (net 3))
 (segment (start 144.5 76) (end 144.5 76.1) (width 0.25) (layer F.Cu) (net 3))
 (segment (start 140.35774 88.61734) (end 138.2 86.4596) (width 0.25) (layer F.Cu) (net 3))
 (segment (start 140.914 88.61734) (end 140.35774 88.61734) (width 0.25) (layer F.Cu) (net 3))
 (segment (start 168.219 88.5996) (end 169.87 88.5996) (width 0.25) (layer F.Cu) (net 3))
 (segment (start 169.87 89.5546) (end 171.267 90.9516) (width 0.25) (layer F.Cu) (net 3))
 (segment (start 170.068 88.7976) (end 169.87 88.5996) (width 0.25) (layer F.Cu) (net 3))
 (segment (start 171.689 88.7976) (end 170.068 88.7976) (width 0.25) (layer F.Cu) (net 3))
 (segment (start 162.5011 74.5236) (end 167.2336 74.5236) (width 0.25) (layer F.Cu) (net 4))
 (segment (start 167.2336 74.5236) (end 167.64 74.93) (width 0.25) (layer F.Cu) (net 4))
 (segment (start 162.5011 76.5236) (end 165.8764 76.5236) (width 0.25) (layer F.Cu) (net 5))
 (segment (start 168.91 76.2) (end 170.18 74.93) (width 0.25) (layer F.Cu) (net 5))
 (segment (start 166.2 76.2) (end 168.91 76.2) (width 0.25) (layer F.Cu) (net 5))
 (segment (start 165.8764 76.5236) (end 166.2 76.2) (width 0.25) (layer F.Cu) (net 5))
 (via (at 171.437 80.0296) (size 0.6) (drill 0.4) (layers F.Cu B.Cu) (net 6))
 (segment (start 161.361 81.0456) (end 161.361 78.1246) (width 0.25) (layer F.Cu) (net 6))
 (segment (start 161.361 78.1246) (end 161.996 77.4896) (width 0.25) (layer F.Cu) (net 6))
 (segment (start 161.996 77.4896) (end 165.425 77.4896) (width 0.25) (layer F.Cu) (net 6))
 (segment (start 165.425 77.4896) (end 167.965 80.0296) (width 0.25) (layer F.Cu) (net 6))
 (segment (start 167.965 80.0296) (end 171.437 80.0296) (width 0.25) (layer F.Cu) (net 6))
 (segment (start 162.5011 82.1857) (end 161.361 81.0456) (width 0.25) (layer F.Cu) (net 6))
 (segment (start 170.18 78.7726) (end 170.18 77.47) (width 0.25) (layer B.Cu) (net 6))
 (segment (start 171.437 80.0296) (end 170.18 78.7726) (width 0.25) (layer B.Cu) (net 6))
 (segment (start 162.5011 82.5236) (end 162.5011 82.1857) (width 0.25) (layer F.Cu) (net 6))
 (segment (start 162.5011 82.5236) (end 162.5011 82.4397) (width 0.25) (layer F.Cu) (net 6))
 (segment (start 170.18 77.9416) (end 170.18 77.47) (width 0.25) (layer F.Cu) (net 6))
 (segment (start 174.696 74.9496) (end 174.696 75.494) (width 0.25) (layer F.Cu) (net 7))
 (segment (start 150.312 72.9176) (end 173.299 72.9176) (width 0.25) (layer F.Cu) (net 7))
 (segment (start 173.299 72.9176) (end 174.696 74.3146) (width 0.25) (layer F.Cu) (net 7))
 (segment (start 174.696 74.3146) (end 174.696 74.9496) (width 0.25) (layer F.Cu) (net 7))
 (segment (start 148.706 74.5236) (end 150.312 72.9176) (width 0.25) (layer F.Cu) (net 7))
 (segment (start 174.696 75.494) (end 172.72 77.47) (width 0.25) (layer F.Cu) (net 7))
 (segment (start 148.5011 74.5236) (end 148.706 74.5236) (width 0.25) (layer F.Cu) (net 7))
 (segment (start 148.5011 74.5236) (end 149.6 75.6225) (width 0.25) (layer F.Cu) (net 7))
 (segment (start 149.6 75.6225) (end 149.6 79.5986) (width 0.25) (layer F.Cu) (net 7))
 (segment (start 149.6 79.5986) (end 148.675 80.5236) (width 0.25) (layer F.Cu) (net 7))
 (segment (start 148.675 80.5236) (end 148.5011 80.5236) (width 0.25) (layer F.Cu) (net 7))
 (segment (start 144.5 74.4) (end 148.3775 74.4) (width 0.25) (layer F.Cu) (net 7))
 (segment (start 148.3775 74.4) (end 148.5011 74.5236) (width 0.25) (layer F.Cu) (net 7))
 (segment (start 148.5011 78.5236) (end 146.992 78.5236) (width 0.25) (layer F.Cu) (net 9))
 (segment (start 146.992 78.5236) (end 144.724 80.7916) (width 0.25) (layer F.Cu) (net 9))
 (segment (start 144.724 80.7916) (end 144.724 82.8666) (width 0.25) (layer F.Cu) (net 9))
 (segment (start 148.5011 78.5236) (end 147.0236 78.5236) (width 0.25) (layer F.Cu) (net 9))
 (segment (start 162.5011 86.5236) (end 166.034 86.5236) (width 0.25) (layer F.Cu) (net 13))
 (segment (start 166.034 86.5236) (end 166.06 86.5496) (width 0.25) (layer F.Cu) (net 13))
 (segment (start 141.549 74.1036) (end 143.327 74.1036) (width 0.25) (layer F.Cu) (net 8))
 (segment (start 143.327 74.1036) (end 144.343 75.1196) (width 0.25) (layer F.Cu) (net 8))
 (segment (start 144.343 75.1196) (end 145.656 75.1196) (width 0.25) (layer F.Cu) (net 8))
 (segment (start 145.656 75.1196) (end 147.06 76.5236) (width 0.25) (layer F.Cu) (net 8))
 (segment (start 147.06 76.5236) (end 148.5011 76.5236) (width 0.25) (layer F.Cu) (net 8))
 (segment (start 148.5011 76.5236) (end 146.8236 76.5236) (width 0.25) (layer F.Cu) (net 8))
 (segment (start 128.325 83.575) (end 128.325 82.175) (width 0.25) (layer F.Cu) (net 17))
 (segment (start 128.325 82.175) (end 128.25 82.1) (width 0.25) (layer F.Cu) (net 17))
 (segment (start 130.525 83.575) (end 131.99 83.575) (width 0.25) (layer F.Cu) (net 18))
 (segment (start 131.99 83.575) (end 132.79 82.775) (width 0.25) (layer F.Cu) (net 18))
 (segment (start 128.65 79.8) (end 128.25 80.2) (width 0.25) (layer F.Cu) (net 18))
 (segment (start 131.6 79.8) (end 128.65 79.8) (width 0.25) (layer F.Cu) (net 18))
 (segment (start 131.6 81.585) (end 132.79 82.775) (width 0.25) (layer F.Cu) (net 18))
 (segment (start 131.6 79.8) (end 131.6 81.585) (width 0.25) (layer F.Cu) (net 18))
 (segment (start 128.325 86) (end 128.4 86) (width 0.25) (layer F.Cu) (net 19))
 (segment (start 128.4 86) (end 129.5 87.1) (width 0.25) (layer F.Cu) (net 19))
 (segment (start 128.325 85.475) (end 128.325 86) (width 0.25) (layer F.Cu) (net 19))
 (segment (start 128.325 86) (end 128.325 86.675) (width 0.25) (layer F.Cu) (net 19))
 (segment (start 128.325 86.675) (end 127.9 87.1) (width 0.25) (layer F.Cu) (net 19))
 (segment (start 127.5 87.1) (end 129.3 87.1) (width 0.25) (layer F.Cu) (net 19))
 (segment (start 131.1 87.1) (end 131.1 86.05) (width 0.25) (layer F.Cu) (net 20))
 (segment (start 131.1 86.05) (end 130.525 85.475) (width 0.25) (layer F.Cu) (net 20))
 (segment (start 171.437 81.6806) (end 168.092 81.6806) (width 0.25) (layer F.Cu) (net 16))
 (segment (start 164.935 78.5236) (end 162.5011 78.5236) (width 0.25) (layer F.Cu) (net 16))
 (segment (start 168.092 81.6806) (end 164.935 78.5236) (width 0.25) (layer F.Cu) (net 16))
 (segment (start 173.639 86.2476) (end 173.639 85.0686) (width 0.25) (layer F.Cu) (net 16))
 (segment (start 172.41 82.6536) (end 171.437 81.6806) (width 0.25) (layer F.Cu) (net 16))
 (segment (start 172.41 83.8396) (end 172.41 82.6536) (width 0.25) (layer F.Cu) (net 16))
 (segment (start 173.639 85.0686) (end 172.41 83.8396) (width 0.25) (layer F.Cu) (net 16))
 (segment (start 163.919 78.5236) (end 162.5011 78.5236) (width 0.25) (layer F.Cu) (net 16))
 (segment (start 171.437 83.3316) (end 168.219 83.3316) (width 0.25) (layer F.Cu) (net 15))
 (segment (start 165.411 80.5236) (end 162.5011 80.5236) (width 0.25) (layer F.Cu) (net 15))
 (segment (start 168.219 83.3316) (end 165.411 80.5236) (width 0.25) (layer F.Cu) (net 15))
 (segment (start 172.989 86.2476) (end 172.989 85.4346) (width 0.25) (layer F.Cu) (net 15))
 (segment (start 171.437 83.8826) (end 171.437 83.3316) (width 0.25) (layer F.Cu) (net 15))
 (segment (start 172.989 85.4346) (end 171.437 83.8826) (width 0.25) (layer F.Cu) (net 15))
 (segment (start 163.647 80.5376) (end 163.633 80.5236) (width 0.25) (layer F.Cu) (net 15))
 (segment (start 163.633 80.5236) (end 162.5011 80.5236) (width 0.25) (layer F.Cu) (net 15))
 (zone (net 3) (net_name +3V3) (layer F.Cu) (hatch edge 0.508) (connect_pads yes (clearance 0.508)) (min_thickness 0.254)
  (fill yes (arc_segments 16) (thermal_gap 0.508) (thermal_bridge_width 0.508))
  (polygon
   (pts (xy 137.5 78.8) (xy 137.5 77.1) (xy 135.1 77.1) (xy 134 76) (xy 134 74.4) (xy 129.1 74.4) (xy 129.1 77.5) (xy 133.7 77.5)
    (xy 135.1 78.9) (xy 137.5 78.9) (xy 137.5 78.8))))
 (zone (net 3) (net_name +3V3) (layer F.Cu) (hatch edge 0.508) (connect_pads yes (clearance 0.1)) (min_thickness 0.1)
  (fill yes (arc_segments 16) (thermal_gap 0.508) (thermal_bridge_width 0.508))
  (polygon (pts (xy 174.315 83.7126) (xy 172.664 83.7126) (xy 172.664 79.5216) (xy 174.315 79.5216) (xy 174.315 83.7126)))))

